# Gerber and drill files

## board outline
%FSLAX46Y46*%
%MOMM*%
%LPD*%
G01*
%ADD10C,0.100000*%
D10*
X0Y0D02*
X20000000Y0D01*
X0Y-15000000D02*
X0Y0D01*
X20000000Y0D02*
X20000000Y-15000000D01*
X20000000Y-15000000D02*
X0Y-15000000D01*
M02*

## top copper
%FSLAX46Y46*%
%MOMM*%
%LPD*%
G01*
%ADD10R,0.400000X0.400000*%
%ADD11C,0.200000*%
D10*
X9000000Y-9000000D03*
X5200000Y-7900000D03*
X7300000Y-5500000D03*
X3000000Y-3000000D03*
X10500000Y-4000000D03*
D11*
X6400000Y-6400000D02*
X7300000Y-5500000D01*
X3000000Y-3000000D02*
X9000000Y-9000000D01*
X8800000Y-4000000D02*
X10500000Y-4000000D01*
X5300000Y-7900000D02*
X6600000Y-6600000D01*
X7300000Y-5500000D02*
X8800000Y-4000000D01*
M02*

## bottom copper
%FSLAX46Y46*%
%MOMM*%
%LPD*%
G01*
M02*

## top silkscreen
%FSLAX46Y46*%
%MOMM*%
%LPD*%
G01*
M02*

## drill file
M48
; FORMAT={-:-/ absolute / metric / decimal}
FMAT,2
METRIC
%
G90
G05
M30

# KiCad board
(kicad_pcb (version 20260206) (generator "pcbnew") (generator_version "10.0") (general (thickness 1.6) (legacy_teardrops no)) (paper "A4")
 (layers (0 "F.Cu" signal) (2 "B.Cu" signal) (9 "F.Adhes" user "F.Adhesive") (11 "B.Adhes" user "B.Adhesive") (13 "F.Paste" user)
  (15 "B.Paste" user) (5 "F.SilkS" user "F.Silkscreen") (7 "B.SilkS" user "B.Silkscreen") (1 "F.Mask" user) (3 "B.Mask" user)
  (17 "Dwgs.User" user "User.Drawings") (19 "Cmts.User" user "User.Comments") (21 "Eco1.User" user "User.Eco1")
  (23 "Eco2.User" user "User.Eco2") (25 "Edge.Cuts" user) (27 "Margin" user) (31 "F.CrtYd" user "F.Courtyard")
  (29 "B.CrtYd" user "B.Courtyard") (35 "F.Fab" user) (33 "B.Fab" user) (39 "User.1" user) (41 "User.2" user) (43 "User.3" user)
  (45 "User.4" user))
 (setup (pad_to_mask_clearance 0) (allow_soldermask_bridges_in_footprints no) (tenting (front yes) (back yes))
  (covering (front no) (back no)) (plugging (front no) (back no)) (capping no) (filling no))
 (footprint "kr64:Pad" (layer "F.Cu") (at 9 9)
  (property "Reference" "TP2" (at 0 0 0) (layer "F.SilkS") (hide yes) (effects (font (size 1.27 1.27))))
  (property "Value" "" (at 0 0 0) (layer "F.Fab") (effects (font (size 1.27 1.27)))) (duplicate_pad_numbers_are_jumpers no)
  (pad "1" smd rect (at 0 0) (size 0.4 0.4) (layers "F.Cu" "F.Mask" "F.Paste") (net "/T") (thermal_bridge_angle 45)))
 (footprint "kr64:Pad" (layer "F.Cu") (at 5.2 7.9)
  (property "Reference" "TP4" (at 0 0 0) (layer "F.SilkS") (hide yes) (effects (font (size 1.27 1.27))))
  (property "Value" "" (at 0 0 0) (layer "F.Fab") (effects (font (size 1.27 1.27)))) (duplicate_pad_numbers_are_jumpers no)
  (pad "1" smd rect (at 0 0) (size 0.4 0.4) (layers "F.Cu" "F.Mask" "F.Paste") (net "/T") (thermal_bridge_angle 45)))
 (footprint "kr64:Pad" (layer "F.Cu") (at 7.3 5.5)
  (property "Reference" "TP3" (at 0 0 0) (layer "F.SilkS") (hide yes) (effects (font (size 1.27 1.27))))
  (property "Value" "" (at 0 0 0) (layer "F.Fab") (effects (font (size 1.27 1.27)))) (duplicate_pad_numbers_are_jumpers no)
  (pad "1" smd rect (at 0 0) (size 0.4 0.4) (layers "F.Cu" "F.Mask" "F.Paste") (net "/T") (thermal_bridge_angle 45)))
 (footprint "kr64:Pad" (layer "F.Cu") (at 3 3)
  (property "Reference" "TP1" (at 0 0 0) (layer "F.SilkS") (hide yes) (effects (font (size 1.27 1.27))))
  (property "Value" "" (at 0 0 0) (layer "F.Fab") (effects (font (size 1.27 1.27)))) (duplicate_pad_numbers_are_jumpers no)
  (pad "1" smd rect (at 0 0) (size 0.4 0.4) (layers "F.Cu" "F.Mask" "F.Paste") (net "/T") (thermal_bridge_angle 45)))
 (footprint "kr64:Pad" (layer "F.Cu") (at 10.5 4)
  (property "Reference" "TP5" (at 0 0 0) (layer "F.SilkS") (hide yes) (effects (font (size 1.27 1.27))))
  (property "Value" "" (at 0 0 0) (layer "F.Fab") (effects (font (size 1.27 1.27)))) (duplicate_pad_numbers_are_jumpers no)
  (pad "1" smd rect (at 0 0) (size 0.4 0.4) (layers "F.Cu" "F.Mask" "F.Paste") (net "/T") (thermal_bridge_angle 45)))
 (gr_line (start 0 0) (end 20 0) (stroke (width 0.1) (type default)) (layer "Edge.Cuts"))
 (gr_line (start 0 15) (end 0 0) (stroke (width 0.1) (type default)) (layer "Edge.Cuts"))
 (gr_line (start 20 0) (end 20 15) (stroke (width 0.1) (type default)) (layer "Edge.Cuts"))
 (gr_line (start 20 15) (end 0 15) (stroke (width 0.1) (type default)) (layer "Edge.Cuts"))
 (segment (start 6.4 6.4) (end 7.3 5.5) (width 0.2) (layer "F.Cu") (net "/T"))
 (segment (start 3 3) (end 9 9) (width 0.2) (layer "F.Cu") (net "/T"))
 (segment (start 8.8 4) (end 10.5 4) (width 0.2) (layer "F.Cu") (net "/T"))
 (segment (start 5.3 7.9) (end 6.6 6.6) (width 0.2) (layer "F.Cu") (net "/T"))
 (segment (start 7.3 5.5) (end 8.8 4) (width 0.2) (layer "F.Cu") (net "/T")))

